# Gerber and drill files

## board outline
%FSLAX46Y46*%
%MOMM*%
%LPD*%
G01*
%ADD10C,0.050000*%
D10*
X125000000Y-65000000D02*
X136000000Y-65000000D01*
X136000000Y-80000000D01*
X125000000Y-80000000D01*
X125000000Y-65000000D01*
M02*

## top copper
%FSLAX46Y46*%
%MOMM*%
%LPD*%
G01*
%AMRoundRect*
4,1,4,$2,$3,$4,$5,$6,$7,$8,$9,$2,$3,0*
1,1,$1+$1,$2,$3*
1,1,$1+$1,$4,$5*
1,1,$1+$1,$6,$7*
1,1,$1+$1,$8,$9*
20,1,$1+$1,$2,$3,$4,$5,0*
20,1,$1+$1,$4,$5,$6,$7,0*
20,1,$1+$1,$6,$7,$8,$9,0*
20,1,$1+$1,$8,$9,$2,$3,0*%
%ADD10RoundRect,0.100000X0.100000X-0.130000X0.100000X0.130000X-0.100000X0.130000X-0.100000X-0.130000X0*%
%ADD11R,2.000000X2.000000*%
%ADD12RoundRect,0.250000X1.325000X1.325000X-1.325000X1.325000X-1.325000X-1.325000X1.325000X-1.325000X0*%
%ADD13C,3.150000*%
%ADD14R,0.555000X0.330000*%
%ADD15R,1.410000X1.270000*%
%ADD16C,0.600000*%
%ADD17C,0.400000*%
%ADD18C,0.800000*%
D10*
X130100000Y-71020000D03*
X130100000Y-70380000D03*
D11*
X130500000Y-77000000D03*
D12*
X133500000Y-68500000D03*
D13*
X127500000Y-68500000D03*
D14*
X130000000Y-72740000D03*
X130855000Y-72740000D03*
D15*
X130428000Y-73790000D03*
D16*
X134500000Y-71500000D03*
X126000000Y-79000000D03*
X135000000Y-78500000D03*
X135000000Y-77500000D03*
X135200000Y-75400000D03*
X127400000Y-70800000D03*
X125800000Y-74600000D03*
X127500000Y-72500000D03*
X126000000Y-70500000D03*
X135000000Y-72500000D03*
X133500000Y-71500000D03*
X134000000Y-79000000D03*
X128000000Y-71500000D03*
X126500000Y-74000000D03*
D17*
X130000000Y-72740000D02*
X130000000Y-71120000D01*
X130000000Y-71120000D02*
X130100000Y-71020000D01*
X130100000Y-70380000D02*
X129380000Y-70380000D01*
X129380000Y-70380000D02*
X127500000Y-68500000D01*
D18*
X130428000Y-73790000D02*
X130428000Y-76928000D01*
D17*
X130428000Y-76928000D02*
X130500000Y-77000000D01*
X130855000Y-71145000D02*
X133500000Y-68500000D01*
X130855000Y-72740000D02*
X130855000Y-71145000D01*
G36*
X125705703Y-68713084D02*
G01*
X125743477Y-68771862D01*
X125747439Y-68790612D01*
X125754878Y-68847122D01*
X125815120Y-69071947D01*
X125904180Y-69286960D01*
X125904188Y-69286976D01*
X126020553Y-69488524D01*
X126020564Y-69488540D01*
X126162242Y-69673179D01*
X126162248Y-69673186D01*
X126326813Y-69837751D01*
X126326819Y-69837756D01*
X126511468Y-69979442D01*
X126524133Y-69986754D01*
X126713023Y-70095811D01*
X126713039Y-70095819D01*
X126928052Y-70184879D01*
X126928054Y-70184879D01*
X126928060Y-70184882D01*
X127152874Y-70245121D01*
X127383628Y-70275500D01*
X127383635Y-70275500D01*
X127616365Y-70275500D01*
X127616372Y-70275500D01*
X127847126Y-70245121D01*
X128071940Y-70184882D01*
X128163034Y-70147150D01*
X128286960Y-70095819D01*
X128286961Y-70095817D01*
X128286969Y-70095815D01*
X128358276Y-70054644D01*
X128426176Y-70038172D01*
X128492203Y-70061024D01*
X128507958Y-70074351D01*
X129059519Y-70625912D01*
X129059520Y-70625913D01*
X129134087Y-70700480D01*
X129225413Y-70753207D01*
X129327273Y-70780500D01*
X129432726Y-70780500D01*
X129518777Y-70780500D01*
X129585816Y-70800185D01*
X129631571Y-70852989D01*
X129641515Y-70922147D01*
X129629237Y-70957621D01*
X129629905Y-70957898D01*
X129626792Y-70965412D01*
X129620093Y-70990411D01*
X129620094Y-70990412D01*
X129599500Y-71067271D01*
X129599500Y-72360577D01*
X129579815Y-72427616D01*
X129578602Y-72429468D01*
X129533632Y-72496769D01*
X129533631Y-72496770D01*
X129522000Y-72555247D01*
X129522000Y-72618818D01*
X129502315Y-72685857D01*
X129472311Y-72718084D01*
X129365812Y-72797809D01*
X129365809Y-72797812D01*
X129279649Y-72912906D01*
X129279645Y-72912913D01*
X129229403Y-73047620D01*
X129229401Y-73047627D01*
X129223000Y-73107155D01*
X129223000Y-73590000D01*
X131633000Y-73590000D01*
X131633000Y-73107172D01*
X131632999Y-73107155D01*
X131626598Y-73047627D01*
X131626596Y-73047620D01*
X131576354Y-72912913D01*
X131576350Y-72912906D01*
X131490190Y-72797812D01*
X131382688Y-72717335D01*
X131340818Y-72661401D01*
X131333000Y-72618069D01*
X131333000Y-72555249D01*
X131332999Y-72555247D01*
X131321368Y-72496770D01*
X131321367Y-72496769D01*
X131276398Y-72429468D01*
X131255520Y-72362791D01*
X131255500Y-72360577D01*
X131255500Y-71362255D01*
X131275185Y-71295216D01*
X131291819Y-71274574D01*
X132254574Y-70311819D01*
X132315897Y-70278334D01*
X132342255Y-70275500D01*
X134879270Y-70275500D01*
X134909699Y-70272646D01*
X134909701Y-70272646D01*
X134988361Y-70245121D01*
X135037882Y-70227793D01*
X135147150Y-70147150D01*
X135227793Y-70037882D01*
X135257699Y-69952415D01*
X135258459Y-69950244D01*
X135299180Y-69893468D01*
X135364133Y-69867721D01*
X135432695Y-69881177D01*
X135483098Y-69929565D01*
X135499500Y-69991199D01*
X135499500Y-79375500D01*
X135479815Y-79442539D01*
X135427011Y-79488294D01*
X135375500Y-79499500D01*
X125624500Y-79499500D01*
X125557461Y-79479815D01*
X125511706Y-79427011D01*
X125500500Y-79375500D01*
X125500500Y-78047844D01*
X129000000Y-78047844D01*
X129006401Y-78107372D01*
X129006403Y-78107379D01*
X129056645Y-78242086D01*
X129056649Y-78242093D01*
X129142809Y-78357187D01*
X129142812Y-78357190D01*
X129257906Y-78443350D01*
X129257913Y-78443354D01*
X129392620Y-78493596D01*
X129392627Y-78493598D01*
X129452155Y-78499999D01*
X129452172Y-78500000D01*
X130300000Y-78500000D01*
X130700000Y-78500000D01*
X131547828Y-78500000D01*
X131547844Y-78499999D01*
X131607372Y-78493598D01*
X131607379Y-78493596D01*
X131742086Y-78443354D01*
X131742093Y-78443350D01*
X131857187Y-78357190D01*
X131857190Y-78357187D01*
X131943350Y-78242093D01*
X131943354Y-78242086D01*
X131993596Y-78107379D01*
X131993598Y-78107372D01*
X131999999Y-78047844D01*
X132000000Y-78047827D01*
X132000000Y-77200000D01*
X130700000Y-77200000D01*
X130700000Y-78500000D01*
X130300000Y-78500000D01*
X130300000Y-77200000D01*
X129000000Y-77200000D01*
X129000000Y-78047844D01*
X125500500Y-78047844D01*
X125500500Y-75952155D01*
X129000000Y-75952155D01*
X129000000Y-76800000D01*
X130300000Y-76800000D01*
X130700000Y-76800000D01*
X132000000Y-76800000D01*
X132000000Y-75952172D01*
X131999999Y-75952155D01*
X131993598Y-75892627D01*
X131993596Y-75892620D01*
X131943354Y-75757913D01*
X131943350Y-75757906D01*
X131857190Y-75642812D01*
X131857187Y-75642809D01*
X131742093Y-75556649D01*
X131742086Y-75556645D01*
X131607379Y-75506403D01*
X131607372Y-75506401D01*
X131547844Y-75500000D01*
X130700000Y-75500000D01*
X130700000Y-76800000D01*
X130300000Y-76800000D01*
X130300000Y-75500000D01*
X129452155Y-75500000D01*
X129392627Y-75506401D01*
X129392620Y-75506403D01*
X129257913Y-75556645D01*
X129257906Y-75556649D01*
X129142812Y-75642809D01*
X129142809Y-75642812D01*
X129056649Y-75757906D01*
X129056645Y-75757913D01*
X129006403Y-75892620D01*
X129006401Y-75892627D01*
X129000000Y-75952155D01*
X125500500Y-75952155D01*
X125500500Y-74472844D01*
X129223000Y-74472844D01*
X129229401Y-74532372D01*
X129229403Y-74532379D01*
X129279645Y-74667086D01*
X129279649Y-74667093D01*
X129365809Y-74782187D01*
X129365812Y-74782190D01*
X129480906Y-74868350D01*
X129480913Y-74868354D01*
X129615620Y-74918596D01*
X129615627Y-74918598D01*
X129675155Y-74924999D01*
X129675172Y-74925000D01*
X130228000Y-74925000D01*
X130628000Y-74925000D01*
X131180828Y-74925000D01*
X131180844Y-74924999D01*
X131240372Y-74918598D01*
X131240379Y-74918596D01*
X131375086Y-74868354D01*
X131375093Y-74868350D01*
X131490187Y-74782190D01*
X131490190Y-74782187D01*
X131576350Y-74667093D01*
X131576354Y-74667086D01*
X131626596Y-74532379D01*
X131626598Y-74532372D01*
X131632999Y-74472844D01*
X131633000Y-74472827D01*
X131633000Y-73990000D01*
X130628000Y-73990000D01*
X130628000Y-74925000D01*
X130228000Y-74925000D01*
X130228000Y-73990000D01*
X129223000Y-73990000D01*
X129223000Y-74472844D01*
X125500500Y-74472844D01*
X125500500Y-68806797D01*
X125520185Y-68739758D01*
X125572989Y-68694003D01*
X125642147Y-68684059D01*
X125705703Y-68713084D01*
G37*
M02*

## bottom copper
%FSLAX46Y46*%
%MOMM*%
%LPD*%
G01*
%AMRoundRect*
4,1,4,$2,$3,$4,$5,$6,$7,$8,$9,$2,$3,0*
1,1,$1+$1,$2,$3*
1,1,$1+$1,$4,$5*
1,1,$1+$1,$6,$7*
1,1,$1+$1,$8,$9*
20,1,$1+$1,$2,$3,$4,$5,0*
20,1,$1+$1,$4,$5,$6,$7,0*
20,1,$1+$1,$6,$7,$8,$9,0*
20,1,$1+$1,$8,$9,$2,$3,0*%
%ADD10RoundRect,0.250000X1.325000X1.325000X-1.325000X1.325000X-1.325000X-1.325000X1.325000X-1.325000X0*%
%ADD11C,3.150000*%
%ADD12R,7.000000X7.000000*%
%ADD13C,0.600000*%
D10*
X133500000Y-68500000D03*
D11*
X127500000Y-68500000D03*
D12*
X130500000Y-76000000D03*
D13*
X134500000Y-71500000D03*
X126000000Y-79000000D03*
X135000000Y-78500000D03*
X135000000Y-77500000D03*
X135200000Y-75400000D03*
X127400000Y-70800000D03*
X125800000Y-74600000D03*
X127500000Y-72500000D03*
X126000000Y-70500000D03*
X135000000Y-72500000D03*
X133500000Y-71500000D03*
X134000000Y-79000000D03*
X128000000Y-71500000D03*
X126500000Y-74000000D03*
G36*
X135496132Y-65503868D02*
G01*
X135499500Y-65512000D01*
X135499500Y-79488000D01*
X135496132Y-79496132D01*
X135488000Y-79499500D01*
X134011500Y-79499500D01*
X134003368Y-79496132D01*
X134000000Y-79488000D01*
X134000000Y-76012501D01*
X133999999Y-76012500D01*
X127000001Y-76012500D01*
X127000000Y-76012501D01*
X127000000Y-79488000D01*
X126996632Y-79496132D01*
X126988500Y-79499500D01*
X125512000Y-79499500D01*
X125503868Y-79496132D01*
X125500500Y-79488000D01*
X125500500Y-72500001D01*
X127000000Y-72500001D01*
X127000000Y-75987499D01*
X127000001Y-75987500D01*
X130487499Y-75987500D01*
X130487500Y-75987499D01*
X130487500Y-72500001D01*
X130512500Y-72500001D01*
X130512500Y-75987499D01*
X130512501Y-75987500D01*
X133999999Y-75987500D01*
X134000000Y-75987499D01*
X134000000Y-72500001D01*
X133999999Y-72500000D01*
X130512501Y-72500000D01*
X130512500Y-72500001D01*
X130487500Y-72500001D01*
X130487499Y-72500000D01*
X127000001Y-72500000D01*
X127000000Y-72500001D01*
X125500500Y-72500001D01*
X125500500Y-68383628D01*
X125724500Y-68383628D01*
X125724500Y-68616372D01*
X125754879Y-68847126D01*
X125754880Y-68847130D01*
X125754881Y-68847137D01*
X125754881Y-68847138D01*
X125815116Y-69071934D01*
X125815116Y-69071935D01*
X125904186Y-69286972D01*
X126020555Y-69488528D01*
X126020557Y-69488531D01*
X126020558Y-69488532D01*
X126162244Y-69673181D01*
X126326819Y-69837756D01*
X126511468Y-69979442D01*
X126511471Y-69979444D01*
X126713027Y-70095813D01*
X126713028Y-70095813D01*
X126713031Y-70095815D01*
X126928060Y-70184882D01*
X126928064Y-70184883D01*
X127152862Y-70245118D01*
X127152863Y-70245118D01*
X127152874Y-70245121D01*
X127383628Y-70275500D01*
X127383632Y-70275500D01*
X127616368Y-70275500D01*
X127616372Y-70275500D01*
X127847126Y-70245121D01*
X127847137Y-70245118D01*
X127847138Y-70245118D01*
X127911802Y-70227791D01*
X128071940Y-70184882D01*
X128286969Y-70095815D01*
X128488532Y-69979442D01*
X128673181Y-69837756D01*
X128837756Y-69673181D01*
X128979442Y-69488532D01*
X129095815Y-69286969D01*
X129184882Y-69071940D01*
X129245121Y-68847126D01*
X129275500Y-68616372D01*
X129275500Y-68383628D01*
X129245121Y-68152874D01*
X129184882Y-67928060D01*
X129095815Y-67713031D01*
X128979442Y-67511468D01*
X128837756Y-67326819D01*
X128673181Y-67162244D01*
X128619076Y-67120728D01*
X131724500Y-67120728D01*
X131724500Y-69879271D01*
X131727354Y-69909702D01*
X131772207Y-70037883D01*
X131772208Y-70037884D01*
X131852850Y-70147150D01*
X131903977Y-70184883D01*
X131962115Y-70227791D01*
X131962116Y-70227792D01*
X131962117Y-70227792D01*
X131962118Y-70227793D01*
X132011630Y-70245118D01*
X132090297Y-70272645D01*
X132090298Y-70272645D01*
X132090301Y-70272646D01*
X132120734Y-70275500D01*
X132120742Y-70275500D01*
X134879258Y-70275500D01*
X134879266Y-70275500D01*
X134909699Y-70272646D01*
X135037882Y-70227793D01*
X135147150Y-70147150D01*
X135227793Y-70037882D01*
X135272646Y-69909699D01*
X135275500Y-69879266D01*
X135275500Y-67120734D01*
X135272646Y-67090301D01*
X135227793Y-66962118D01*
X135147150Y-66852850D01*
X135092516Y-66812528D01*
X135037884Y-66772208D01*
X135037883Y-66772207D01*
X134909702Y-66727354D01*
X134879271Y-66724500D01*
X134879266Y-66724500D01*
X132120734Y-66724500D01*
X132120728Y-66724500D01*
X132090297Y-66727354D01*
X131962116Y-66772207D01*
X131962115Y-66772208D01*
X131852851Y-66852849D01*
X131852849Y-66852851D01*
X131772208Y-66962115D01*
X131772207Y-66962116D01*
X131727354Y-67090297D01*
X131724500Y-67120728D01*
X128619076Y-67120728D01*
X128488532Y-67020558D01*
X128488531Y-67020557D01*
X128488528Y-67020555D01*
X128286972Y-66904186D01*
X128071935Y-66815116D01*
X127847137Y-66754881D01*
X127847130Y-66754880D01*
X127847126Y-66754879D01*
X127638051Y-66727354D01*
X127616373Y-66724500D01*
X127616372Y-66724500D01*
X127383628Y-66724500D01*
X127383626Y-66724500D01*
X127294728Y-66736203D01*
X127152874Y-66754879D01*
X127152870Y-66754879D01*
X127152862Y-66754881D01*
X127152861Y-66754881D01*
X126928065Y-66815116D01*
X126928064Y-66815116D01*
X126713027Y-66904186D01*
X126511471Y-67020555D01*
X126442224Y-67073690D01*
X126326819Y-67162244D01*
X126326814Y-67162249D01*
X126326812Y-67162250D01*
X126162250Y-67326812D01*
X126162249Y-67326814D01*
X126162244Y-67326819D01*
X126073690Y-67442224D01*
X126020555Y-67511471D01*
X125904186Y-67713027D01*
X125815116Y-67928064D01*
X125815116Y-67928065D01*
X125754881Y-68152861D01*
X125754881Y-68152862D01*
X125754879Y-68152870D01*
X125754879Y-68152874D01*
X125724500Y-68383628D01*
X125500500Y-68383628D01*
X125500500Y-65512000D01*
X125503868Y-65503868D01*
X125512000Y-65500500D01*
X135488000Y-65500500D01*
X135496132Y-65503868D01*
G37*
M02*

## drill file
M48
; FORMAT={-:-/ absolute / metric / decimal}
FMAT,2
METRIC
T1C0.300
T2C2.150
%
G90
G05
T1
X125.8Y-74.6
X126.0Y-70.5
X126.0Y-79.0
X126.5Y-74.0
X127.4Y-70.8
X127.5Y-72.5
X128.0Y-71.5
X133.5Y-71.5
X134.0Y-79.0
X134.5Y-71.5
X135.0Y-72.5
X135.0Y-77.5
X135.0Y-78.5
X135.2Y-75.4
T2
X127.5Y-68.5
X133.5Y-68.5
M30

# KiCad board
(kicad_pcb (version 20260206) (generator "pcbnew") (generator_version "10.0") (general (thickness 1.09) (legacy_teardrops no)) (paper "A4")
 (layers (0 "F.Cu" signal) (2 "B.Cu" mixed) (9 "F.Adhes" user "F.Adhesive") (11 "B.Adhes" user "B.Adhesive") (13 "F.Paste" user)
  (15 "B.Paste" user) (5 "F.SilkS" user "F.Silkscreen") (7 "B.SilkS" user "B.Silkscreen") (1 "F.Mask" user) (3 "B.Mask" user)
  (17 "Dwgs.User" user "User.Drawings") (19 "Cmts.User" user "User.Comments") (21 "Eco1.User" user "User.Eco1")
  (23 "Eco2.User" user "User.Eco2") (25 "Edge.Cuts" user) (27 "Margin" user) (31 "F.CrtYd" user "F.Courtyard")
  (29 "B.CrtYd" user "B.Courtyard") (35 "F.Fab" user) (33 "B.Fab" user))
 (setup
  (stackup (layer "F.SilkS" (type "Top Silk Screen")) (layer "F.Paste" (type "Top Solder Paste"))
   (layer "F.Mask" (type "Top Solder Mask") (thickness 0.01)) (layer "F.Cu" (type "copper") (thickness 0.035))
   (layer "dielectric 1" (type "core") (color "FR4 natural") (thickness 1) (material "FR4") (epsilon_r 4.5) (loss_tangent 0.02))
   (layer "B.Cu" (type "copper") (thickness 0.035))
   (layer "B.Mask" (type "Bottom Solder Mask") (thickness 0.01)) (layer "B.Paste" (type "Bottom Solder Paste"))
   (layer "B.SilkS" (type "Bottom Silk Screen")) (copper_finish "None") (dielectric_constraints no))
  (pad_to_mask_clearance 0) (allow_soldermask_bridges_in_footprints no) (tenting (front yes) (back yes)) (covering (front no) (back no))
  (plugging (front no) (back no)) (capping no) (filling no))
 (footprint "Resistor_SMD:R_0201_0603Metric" (layer "F.Cu") (at 130.1 70.7 90)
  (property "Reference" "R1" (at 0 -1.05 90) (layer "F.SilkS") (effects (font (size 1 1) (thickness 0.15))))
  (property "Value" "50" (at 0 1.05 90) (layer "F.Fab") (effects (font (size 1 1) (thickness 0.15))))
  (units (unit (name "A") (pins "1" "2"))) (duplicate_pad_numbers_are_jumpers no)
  (pad "" smd roundrect (at -0.345 0 90) (size 0.318 0.36) (layers "F.Paste") (roundrect_rratio 0.25))
  (pad "" smd roundrect (at 0.345 0 90) (size 0.318 0.36) (layers "F.Paste") (roundrect_rratio 0.25))
  (pad "1" smd roundrect (at -0.32 0 90) (size 0.46 0.4) (layers "F.Cu" "F.Mask") (roundrect_rratio 0.25) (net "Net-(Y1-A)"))
  (pad "2" smd roundrect (at 0.32 0 90) (size 0.46 0.4) (layers "F.Cu" "F.Mask") (roundrect_rratio 0.25) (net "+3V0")))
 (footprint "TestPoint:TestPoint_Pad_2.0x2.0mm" (layer "F.Cu") (at 130.5 77)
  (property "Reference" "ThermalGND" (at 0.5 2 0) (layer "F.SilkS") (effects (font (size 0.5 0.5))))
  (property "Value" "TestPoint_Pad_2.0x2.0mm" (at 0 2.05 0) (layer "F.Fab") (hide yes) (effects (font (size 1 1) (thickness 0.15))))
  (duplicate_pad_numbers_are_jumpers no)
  (pad "1" smd rect (at 0 0) (size 2 2) (layers "F.Cu" "F.Mask") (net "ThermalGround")))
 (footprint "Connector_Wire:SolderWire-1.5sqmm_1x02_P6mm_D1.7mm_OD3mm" (layer "F.Cu") (at 133.5 68.5 180)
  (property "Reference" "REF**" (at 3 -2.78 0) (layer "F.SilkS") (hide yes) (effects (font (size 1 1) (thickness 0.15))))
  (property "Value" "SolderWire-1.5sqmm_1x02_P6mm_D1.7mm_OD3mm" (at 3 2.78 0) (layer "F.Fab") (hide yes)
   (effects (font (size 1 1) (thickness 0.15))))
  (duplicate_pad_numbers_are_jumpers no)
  (pad "1" thru_hole roundrect (at 0 0 180) (size 3.15 3.15) (drill 2.15) (layers "*.Cu" "*.Mask") (remove_unused_layers no)
   (roundrect_rratio 0.079365) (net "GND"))
  (pad "2" thru_hole circle (at 6 0 180) (size 3.15 3.15) (drill 2.15) (layers "*.Cu" "*.Mask") (remove_unused_layers no) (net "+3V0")))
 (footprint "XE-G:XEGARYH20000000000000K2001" (layer "F.Cu") (at 130.428 73.5)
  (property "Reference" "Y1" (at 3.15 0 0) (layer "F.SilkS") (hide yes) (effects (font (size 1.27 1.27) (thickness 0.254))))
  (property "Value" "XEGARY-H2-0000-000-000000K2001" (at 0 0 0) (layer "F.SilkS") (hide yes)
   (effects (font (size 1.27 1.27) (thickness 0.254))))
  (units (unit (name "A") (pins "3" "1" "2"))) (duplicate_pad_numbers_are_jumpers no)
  (pad "1" smd rect (at -0.428 -0.76 90) (size 0.33 0.555) (layers "F.Cu" "F.Mask" "F.Paste") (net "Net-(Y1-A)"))
  (pad "2" smd rect (at 0.427 -0.76 90) (size 0.33 0.555) (layers "F.Cu" "F.Mask" "F.Paste") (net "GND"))
  (pad "3" smd rect (at 0 0.29 90) (size 1.27 1.41) (layers "F.Cu" "F.Mask" "F.Paste") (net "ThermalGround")))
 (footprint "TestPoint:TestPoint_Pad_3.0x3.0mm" (layer "B.Cu") (at 130.5 76 180)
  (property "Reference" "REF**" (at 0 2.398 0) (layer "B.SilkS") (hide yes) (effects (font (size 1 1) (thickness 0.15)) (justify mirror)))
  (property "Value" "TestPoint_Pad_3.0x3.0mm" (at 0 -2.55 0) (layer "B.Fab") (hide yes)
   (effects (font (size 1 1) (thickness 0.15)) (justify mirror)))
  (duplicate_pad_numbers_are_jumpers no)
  (pad "1" smd rect (at 0 0 180) (size 7 7) (layers "B.Cu" "B.Mask") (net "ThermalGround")))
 (gr_rect (start 125 65) (end 136 80) (stroke (width 0.05) (type default)) (fill no) (layer "Edge.Cuts"))
 (segment (start 130 72.74) (end 130 71.12) (width 0.4) (layer "F.Cu") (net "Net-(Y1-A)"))
 (segment (start 130 71.12) (end 130.1 71.02) (width 0.4) (layer "F.Cu") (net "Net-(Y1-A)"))
 (segment (start 130.1 70.38) (end 129.38 70.38) (width 0.4) (layer "F.Cu") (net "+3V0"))
 (segment (start 129.38 70.38) (end 127.5 68.5) (width 0.4) (layer "F.Cu") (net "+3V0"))
 (segment (start 130.428 73.79) (end 130.428 76.928) (width 0.8) (layer "F.Cu") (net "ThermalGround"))
 (segment (start 130.428 76.928) (end 130.5 77) (width 0.4) (layer "F.Cu") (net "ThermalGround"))
 (via (at 134.5 71.5) (size 0.6) (drill 0.3) (layers "F.Cu" "B.Cu") (free yes) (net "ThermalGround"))
 (via (at 126 79) (size 0.6) (drill 0.3) (layers "F.Cu" "B.Cu") (free yes) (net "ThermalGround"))
 (via (at 135 78.5) (size 0.6) (drill 0.3) (layers "F.Cu" "B.Cu") (free yes) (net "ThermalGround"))
 (via (at 135 77.5) (size 0.6) (drill 0.3) (layers "F.Cu" "B.Cu") (free yes) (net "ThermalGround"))
 (via (at 135.2 75.4) (size 0.6) (drill 0.3) (layers "F.Cu" "B.Cu") (free yes) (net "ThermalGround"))
 (via (at 127.4 70.8) (size 0.6) (drill 0.3) (layers "F.Cu" "B.Cu") (free yes) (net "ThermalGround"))
 (via (at 125.8 74.6) (size 0.6) (drill 0.3) (layers "F.Cu" "B.Cu") (free yes) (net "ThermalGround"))
 (via (at 127.5 72.5) (size 0.6) (drill 0.3) (layers "F.Cu" "B.Cu") (free yes) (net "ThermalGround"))
 (via (at 126 70.5) (size 0.6) (drill 0.3) (layers "F.Cu" "B.Cu") (free yes) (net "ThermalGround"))
 (via (at 135 72.5) (size 0.6) (drill 0.3) (layers "F.Cu" "B.Cu") (free yes) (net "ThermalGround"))
 (via (at 133.5 71.5) (size 0.6) (drill 0.3) (layers "F.Cu" "B.Cu") (free yes) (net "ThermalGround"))
 (via (at 134 79) (size 0.6) (drill 0.3) (layers "F.Cu" "B.Cu") (free yes) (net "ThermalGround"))
 (via (at 128 71.5) (size 0.6) (drill 0.3) (layers "F.Cu" "B.Cu") (free yes) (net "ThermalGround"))
 (via (at 126.5 74) (size 0.6) (drill 0.3) (layers "F.Cu" "B.Cu") (free yes) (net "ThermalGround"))
 (segment (start 130.855 71.145) (end 133.5 68.5) (width 0.4) (layer "F.Cu") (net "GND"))
 (segment (start 130.855 72.74) (end 130.855 71.145) (width 0.4) (layer "F.Cu") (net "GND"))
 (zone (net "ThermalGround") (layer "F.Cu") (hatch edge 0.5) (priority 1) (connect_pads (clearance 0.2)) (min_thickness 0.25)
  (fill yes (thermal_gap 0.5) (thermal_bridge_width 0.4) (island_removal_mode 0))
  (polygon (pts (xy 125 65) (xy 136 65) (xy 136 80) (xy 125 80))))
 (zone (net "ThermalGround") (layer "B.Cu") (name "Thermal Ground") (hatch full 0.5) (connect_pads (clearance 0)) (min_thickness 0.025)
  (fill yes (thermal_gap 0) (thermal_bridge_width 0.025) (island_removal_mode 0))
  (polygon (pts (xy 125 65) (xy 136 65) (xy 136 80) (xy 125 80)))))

